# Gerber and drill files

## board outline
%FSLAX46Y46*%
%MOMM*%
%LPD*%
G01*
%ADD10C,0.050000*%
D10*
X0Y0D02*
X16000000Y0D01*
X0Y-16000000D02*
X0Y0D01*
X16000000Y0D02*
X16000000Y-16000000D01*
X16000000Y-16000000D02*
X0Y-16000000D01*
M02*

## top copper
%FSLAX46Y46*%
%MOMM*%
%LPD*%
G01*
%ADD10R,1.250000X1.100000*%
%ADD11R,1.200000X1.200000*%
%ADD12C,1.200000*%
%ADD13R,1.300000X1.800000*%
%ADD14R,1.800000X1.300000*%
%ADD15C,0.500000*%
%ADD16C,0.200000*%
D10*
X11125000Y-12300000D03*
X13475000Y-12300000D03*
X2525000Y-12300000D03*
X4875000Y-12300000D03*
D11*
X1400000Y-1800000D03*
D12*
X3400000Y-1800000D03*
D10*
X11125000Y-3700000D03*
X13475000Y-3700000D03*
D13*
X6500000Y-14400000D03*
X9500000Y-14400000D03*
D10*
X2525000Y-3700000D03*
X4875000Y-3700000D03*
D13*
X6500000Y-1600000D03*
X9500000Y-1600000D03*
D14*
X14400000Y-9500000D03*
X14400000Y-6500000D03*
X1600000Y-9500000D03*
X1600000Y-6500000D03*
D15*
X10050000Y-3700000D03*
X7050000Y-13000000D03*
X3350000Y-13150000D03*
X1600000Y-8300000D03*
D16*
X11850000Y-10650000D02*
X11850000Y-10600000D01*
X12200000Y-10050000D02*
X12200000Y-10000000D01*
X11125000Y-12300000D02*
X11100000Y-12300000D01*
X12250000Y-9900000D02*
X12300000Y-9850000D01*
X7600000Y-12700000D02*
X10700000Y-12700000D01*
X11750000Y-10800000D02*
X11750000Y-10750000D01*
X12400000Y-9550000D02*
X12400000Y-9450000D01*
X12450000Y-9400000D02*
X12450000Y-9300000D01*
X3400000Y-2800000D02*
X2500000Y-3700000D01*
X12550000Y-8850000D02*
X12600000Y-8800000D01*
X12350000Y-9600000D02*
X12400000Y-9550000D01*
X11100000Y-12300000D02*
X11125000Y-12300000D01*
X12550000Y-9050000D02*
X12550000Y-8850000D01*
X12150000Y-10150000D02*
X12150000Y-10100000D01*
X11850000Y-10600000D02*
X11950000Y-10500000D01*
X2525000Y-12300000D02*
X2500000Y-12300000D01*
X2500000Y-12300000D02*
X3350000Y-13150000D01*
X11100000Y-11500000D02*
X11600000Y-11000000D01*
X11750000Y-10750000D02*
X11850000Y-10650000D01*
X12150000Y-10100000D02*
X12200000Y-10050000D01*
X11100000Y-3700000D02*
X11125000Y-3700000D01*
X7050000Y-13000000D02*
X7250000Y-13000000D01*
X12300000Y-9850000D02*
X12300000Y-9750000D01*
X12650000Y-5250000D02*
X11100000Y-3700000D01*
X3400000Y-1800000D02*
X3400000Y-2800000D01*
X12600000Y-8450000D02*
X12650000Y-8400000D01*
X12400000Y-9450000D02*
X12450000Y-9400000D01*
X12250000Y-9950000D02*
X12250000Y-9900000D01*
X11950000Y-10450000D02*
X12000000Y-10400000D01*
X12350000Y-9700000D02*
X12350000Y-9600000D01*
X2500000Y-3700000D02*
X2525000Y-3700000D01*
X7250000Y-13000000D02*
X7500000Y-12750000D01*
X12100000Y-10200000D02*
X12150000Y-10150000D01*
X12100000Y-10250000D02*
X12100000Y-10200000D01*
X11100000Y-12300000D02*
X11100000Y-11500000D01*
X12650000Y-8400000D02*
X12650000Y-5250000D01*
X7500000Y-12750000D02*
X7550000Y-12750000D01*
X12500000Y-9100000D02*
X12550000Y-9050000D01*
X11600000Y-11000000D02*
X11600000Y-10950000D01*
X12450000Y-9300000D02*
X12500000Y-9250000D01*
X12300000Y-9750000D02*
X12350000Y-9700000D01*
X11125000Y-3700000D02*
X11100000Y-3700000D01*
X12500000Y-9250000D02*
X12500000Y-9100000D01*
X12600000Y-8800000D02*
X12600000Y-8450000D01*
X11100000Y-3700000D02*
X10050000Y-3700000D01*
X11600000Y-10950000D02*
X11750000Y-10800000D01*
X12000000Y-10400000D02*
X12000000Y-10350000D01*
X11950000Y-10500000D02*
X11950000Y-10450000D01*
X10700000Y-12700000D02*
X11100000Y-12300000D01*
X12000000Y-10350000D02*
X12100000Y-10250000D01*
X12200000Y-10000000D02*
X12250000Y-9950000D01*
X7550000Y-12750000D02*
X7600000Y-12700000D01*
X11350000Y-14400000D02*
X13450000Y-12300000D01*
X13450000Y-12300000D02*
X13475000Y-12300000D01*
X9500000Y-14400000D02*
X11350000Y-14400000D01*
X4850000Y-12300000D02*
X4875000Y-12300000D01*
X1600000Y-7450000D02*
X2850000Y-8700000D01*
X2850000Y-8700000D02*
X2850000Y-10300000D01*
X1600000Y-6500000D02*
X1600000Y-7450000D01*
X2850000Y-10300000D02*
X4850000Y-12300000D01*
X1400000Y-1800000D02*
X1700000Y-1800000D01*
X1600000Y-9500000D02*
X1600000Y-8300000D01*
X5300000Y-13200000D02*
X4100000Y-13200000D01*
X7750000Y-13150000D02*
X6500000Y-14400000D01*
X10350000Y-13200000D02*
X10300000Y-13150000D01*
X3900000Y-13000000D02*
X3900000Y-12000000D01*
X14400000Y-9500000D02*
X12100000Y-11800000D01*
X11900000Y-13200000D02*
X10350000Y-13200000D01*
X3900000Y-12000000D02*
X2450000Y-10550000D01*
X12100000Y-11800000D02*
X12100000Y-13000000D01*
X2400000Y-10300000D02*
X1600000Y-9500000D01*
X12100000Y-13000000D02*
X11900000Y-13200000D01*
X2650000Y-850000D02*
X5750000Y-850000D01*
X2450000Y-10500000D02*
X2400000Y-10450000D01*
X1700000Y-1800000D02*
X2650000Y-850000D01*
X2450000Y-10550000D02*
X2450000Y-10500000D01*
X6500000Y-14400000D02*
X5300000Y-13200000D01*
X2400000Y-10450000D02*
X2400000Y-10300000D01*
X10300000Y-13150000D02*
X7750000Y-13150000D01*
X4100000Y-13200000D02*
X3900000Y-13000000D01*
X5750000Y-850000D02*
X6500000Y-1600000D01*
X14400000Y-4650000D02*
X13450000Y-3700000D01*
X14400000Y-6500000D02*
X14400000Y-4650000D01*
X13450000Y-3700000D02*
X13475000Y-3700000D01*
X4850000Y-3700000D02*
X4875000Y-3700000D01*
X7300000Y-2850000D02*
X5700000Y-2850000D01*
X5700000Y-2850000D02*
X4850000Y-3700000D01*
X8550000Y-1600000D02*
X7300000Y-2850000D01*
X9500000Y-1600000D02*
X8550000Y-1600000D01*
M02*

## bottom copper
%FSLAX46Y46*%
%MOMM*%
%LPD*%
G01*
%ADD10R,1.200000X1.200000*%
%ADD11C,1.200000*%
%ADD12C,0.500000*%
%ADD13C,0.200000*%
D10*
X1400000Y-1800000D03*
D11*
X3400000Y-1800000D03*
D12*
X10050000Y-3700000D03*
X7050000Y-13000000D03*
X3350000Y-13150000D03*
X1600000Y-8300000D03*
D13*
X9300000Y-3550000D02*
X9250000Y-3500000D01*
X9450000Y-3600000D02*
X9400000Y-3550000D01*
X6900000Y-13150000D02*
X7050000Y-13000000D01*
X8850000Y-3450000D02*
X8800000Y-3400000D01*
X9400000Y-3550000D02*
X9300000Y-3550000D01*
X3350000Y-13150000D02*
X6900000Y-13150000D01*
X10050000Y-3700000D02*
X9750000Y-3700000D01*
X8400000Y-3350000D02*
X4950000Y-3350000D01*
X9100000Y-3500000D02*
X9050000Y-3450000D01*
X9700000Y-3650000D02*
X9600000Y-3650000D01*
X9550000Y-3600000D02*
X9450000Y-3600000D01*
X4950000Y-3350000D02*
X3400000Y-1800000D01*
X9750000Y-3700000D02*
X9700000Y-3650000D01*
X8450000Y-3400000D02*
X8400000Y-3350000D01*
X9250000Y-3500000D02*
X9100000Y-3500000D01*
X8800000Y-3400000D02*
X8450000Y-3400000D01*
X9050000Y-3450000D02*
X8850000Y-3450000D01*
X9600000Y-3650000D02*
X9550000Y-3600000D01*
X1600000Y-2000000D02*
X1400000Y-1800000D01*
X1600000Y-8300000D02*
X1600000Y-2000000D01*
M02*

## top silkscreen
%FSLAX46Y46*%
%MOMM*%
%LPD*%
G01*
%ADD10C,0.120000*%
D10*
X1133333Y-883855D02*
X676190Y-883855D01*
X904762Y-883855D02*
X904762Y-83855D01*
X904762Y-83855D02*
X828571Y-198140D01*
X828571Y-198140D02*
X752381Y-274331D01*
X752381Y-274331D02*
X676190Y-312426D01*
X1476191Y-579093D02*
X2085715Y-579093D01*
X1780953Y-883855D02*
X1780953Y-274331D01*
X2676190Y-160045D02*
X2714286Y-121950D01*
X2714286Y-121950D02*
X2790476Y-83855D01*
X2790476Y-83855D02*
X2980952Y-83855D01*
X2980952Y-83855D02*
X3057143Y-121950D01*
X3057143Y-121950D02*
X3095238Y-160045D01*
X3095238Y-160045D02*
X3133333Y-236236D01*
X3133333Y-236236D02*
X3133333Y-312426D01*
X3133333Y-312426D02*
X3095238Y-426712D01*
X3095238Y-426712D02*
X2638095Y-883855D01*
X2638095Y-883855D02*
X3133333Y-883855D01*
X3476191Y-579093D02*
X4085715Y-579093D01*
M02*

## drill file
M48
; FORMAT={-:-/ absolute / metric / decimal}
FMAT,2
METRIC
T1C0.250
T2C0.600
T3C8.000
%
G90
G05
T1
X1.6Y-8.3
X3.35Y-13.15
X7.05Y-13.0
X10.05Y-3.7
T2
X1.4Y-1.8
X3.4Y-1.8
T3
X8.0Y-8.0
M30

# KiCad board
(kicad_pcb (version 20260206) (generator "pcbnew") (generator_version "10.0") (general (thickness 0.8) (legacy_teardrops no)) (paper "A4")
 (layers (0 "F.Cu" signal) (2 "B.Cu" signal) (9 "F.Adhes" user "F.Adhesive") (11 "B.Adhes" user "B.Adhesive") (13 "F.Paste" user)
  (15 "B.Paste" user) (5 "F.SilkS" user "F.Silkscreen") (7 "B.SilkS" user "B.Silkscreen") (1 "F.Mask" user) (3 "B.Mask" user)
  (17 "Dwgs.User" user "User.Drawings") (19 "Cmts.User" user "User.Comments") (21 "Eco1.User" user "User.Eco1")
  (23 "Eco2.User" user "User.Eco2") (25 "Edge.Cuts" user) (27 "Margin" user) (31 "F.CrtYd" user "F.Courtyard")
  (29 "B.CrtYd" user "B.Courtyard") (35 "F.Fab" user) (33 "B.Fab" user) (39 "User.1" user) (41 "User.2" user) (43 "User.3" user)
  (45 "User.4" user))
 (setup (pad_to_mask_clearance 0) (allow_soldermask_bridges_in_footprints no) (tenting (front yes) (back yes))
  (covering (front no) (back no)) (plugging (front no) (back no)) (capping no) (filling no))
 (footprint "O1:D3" (layer "F.Cu") (at 12.3 12.3)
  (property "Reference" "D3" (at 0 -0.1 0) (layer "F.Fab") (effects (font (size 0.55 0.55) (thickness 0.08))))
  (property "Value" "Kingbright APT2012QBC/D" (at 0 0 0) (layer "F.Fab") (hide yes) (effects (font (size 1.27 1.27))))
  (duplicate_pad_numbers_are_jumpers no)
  (pad "1" smd rect (at -1.175 0) (size 1.25 1.1) (layers "F.Cu" "F.Mask" "F.Paste") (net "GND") (solder_mask_margin 0.025)
   (thermal_bridge_angle 45))
  (pad "2" smd rect (at 1.175 0) (size 1.25 1.1) (layers "F.Cu" "F.Mask" "F.Paste") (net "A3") (solder_mask_margin 0.025)
   (thermal_bridge_angle 45)))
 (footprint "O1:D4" (layer "F.Cu") (at 3.7 12.3)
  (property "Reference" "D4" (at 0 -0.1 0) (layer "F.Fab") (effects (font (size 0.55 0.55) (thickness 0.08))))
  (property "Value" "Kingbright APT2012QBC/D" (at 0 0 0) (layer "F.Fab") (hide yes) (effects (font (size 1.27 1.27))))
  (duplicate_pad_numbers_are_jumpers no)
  (pad "1" smd rect (at -1.175 0) (size 1.25 1.1) (layers "F.Cu" "F.Mask" "F.Paste") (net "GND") (solder_mask_margin 0.025)
   (thermal_bridge_angle 45))
  (pad "2" smd rect (at 1.175 0) (size 1.25 1.1) (layers "F.Cu" "F.Mask" "F.Paste") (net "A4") (solder_mask_margin 0.025)
   (thermal_bridge_angle 45)))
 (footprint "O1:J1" (layer "F.Cu") (at 2.4 1.8)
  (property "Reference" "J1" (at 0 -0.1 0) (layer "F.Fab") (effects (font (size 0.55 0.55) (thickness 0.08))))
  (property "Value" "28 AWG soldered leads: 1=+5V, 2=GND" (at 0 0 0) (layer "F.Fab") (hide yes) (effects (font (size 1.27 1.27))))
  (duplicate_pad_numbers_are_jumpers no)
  (pad "1" thru_hole rect (at -1 0) (size 1.2 1.2) (drill 0.6) (layers "*.Cu" "*.Mask") (remove_unused_layers no) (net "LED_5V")
   (solder_mask_margin 0.025) (thermal_bridge_angle 45))
  (pad "2" thru_hole circle (at 1 0) (size 1.2 1.2) (drill 0.6) (layers "*.Cu" "*.Mask") (remove_unused_layers no) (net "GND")
   (solder_mask_margin 0.025)))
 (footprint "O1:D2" (layer "F.Cu") (at 12.3 3.7)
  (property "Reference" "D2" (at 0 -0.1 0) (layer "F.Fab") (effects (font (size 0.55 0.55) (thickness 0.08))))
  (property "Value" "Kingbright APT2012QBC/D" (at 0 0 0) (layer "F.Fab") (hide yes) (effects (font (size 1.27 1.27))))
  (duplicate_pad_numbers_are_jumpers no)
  (pad "1" smd rect (at -1.175 0) (size 1.25 1.1) (layers "F.Cu" "F.Mask" "F.Paste") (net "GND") (solder_mask_margin 0.025)
   (thermal_bridge_angle 45))
  (pad "2" smd rect (at 1.175 0) (size 1.25 1.1) (layers "F.Cu" "F.Mask" "F.Paste") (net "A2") (solder_mask_margin 0.025)
   (thermal_bridge_angle 45)))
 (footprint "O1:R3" (layer "F.Cu") (at 8 14.4)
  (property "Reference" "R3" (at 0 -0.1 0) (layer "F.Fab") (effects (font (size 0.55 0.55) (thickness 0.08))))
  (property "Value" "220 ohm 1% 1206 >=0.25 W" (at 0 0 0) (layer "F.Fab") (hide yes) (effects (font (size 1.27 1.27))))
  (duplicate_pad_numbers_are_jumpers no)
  (pad "1" smd rect (at -1.5 0) (size 1.3 1.8) (layers "F.Cu" "F.Mask" "F.Paste") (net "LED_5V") (solder_mask_margin 0.025)
   (thermal_bridge_angle 45))
  (pad "2" smd rect (at 1.5 0) (size 1.3 1.8) (layers "F.Cu" "F.Mask" "F.Paste") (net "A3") (solder_mask_margin 0.025)
   (thermal_bridge_angle 45)))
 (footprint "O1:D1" (layer "F.Cu") (at 3.7 3.7)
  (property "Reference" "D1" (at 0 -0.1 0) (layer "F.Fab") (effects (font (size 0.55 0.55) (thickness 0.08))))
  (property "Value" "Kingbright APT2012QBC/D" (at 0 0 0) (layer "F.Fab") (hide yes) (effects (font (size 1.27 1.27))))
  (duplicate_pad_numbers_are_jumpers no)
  (pad "1" smd rect (at -1.175 0) (size 1.25 1.1) (layers "F.Cu" "F.Mask" "F.Paste") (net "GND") (solder_mask_margin 0.025)
   (thermal_bridge_angle 45))
  (pad "2" smd rect (at 1.175 0) (size 1.25 1.1) (layers "F.Cu" "F.Mask" "F.Paste") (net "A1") (solder_mask_margin 0.025)
   (thermal_bridge_angle 45)))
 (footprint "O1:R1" (layer "F.Cu") (at 8 1.6)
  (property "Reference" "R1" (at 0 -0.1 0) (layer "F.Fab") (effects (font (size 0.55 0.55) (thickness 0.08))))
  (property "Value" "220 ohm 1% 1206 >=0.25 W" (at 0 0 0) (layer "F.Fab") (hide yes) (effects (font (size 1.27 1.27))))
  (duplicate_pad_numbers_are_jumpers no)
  (pad "1" smd rect (at -1.5 0) (size 1.3 1.8) (layers "F.Cu" "F.Mask" "F.Paste") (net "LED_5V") (solder_mask_margin 0.025)
   (thermal_bridge_angle 45))
  (pad "2" smd rect (at 1.5 0) (size 1.3 1.8) (layers "F.Cu" "F.Mask" "F.Paste") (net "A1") (solder_mask_margin 0.025)
   (thermal_bridge_angle 45)))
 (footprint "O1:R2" (layer "F.Cu") (at 14.4 8 90)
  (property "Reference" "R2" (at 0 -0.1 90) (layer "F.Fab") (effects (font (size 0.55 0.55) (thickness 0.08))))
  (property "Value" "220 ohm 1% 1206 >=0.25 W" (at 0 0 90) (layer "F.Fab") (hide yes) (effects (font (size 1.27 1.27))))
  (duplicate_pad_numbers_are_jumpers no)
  (pad "1" smd rect (at -1.5 0 90) (size 1.3 1.8) (layers "F.Cu" "F.Mask" "F.Paste") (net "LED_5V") (solder_mask_margin 0.025)
   (thermal_bridge_angle 45))
  (pad "2" smd rect (at 1.5 0 90) (size 1.3 1.8) (layers "F.Cu" "F.Mask" "F.Paste") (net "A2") (solder_mask_margin 0.025)
   (thermal_bridge_angle 45)))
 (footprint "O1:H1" (layer "F.Cu") (at 8 8)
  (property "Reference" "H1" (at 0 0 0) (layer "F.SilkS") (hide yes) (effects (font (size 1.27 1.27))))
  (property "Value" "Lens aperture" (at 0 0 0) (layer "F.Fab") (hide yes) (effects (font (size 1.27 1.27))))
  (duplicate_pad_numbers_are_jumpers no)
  (pad "" np_thru_hole circle (at 0 0) (size 8 8) (drill 8) (layers "*.Cu" "*.Mask")))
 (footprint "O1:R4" (layer "F.Cu") (at 1.6 8 90)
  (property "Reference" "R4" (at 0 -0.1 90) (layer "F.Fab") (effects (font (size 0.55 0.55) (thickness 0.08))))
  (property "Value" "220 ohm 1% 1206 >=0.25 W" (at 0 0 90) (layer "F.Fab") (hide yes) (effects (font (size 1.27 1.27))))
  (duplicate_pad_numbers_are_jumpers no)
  (pad "1" smd rect (at -1.5 0 90) (size 1.3 1.8) (layers "F.Cu" "F.Mask" "F.Paste") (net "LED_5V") (solder_mask_margin 0.025)
   (thermal_bridge_angle 45))
  (pad "2" smd rect (at 1.5 0 90) (size 1.3 1.8) (layers "F.Cu" "F.Mask" "F.Paste") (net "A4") (solder_mask_margin 0.025)
   (thermal_bridge_angle 45)))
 (gr_line (start 0 0) (end 16 0) (stroke (width 0.05) (type default)) (layer "Edge.Cuts"))
 (gr_line (start 0 16) (end 0 0) (stroke (width 0.05) (type default)) (layer "Edge.Cuts"))
 (gr_line (start 16 0) (end 16 16) (stroke (width 0.05) (type default)) (layer "Edge.Cuts"))
 (gr_line (start 16 16) (end 0 16) (stroke (width 0.05) (type default)) (layer "Edge.Cuts"))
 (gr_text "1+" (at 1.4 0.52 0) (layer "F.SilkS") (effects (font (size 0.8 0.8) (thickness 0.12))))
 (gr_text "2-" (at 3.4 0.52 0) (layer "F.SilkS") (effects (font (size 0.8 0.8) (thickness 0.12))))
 (segment (start 11.85 10.65) (end 11.85 10.6) (width 0.2) (layer "F.Cu") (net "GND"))
 (segment (start 12.2 10.05) (end 12.2 10) (width 0.2) (layer "F.Cu") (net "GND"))
 (segment (start 11.125 12.3) (end 11.1 12.3) (width 0.2) (layer "F.Cu") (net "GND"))
 (segment (start 12.25 9.9) (end 12.3 9.85) (width 0.2) (layer "F.Cu") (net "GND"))
 (segment (start 7.6 12.7) (end 10.7 12.7) (width 0.2) (layer "F.Cu") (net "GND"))
 (segment (start 11.75 10.8) (end 11.75 10.75) (width 0.2) (layer "F.Cu") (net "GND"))
 (segment (start 12.4 9.55) (end 12.4 9.45) (width 0.2) (layer "F.Cu") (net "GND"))
 (segment (start 12.45 9.4) (end 12.45 9.3) (width 0.2) (layer "F.Cu") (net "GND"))
 (segment (start 3.4 2.8) (end 2.5 3.7) (width 0.2) (layer "F.Cu") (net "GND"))
 (segment (start 12.55 8.85) (end 12.6 8.8) (width 0.2) (layer "F.Cu") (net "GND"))
 (segment (start 12.35 9.6) (end 12.4 9.55) (width 0.2) (layer "F.Cu") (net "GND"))
 (segment (start 11.1 12.3) (end 11.125 12.3) (width 0.2) (layer "F.Cu") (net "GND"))
 (segment (start 12.55 9.05) (end 12.55 8.85) (width 0.2) (layer "F.Cu") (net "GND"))
 (segment (start 12.15 10.15) (end 12.15 10.1) (width 0.2) (layer "F.Cu") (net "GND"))
 (segment (start 11.85 10.6) (end 11.95 10.5) (width 0.2) (layer "F.Cu") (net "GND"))
 (segment (start 2.525 12.3) (end 2.5 12.3) (width 0.2) (layer "F.Cu") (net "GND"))
 (segment (start 2.5 12.3) (end 3.35 13.15) (width 0.2) (layer "F.Cu") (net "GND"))
 (segment (start 11.1 11.5) (end 11.6 11) (width 0.2) (layer "F.Cu") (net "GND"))
 (segment (start 11.75 10.75) (end 11.85 10.65) (width 0.2) (layer "F.Cu") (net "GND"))
 (segment (start 12.15 10.1) (end 12.2 10.05) (width 0.2) (layer "F.Cu") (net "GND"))
 (segment (start 11.1 3.7) (end 11.125 3.7) (width 0.2) (layer "F.Cu") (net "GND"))
 (segment (start 7.05 13) (end 7.25 13) (width 0.2) (layer "F.Cu") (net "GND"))
 (segment (start 12.3 9.85) (end 12.3 9.75) (width 0.2) (layer "F.Cu") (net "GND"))
 (segment (start 12.65 5.25) (end 11.1 3.7) (width 0.2) (layer "F.Cu") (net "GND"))
 (segment (start 3.4 1.8) (end 3.4 2.8) (width 0.2) (layer "F.Cu") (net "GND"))
 (segment (start 12.6 8.45) (end 12.65 8.4) (width 0.2) (layer "F.Cu") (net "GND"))
 (segment (start 12.4 9.45) (end 12.45 9.4) (width 0.2) (layer "F.Cu") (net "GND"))
 (segment (start 12.25 9.95) (end 12.25 9.9) (width 0.2) (layer "F.Cu") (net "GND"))
 (segment (start 11.95 10.45) (end 12 10.4) (width 0.2) (layer "F.Cu") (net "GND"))
 (segment (start 12.35 9.7) (end 12.35 9.6) (width 0.2) (layer "F.Cu") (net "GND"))
 (segment (start 2.5 3.7) (end 2.525 3.7) (width 0.2) (layer "F.Cu") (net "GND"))
 (segment (start 7.25 13) (end 7.5 12.75) (width 0.2) (layer "F.Cu") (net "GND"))
 (segment (start 12.1 10.2) (end 12.15 10.15) (width 0.2) (layer "F.Cu") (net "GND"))
 (segment (start 12.1 10.25) (end 12.1 10.2) (width 0.2) (layer "F.Cu") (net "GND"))
 (segment (start 11.1 12.3) (end 11.1 11.5) (width 0.2) (layer "F.Cu") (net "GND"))
 (segment (start 12.65 8.4) (end 12.65 5.25) (width 0.2) (layer "F.Cu") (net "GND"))
 (segment (start 7.5 12.75) (end 7.55 12.75) (width 0.2) (layer "F.Cu") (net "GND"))
 (segment (start 12.5 9.1) (end 12.55 9.05) (width 0.2) (layer "F.Cu") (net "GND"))
 (segment (start 11.6 11) (end 11.6 10.95) (width 0.2) (layer "F.Cu") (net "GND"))
 (segment (start 12.45 9.3) (end 12.5 9.25) (width 0.2) (layer "F.Cu") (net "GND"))
 (segment (start 12.3 9.75) (end 12.35 9.7) (width 0.2) (layer "F.Cu") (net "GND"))
 (segment (start 11.125 3.7) (end 11.1 3.7) (width 0.2) (layer "F.Cu") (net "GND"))
 (segment (start 12.5 9.25) (end 12.5 9.1) (width 0.2) (layer "F.Cu") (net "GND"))
 (segment (start 12.6 8.8) (end 12.6 8.45) (width 0.2) (layer "F.Cu") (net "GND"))
 (segment (start 11.1 3.7) (end 10.05 3.7) (width 0.2) (layer "F.Cu") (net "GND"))
 (segment (start 11.6 10.95) (end 11.75 10.8) (width 0.2) (layer "F.Cu") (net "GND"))
 (segment (start 12 10.4) (end 12 10.35) (width 0.2) (layer "F.Cu") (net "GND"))
 (segment (start 11.95 10.5) (end 11.95 10.45) (width 0.2) (layer "F.Cu") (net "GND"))
 (segment (start 10.7 12.7) (end 11.1 12.3) (width 0.2) (layer "F.Cu") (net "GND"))
 (segment (start 12 10.35) (end 12.1 10.25) (width 0.2) (layer "F.Cu") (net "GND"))
 (segment (start 12.2 10) (end 12.25 9.95) (width 0.2) (layer "F.Cu") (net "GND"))
 (segment (start 7.55 12.75) (end 7.6 12.7) (width 0.2) (layer "F.Cu") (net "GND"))
 (via (at 10.05 3.7) (size 0.5) (drill 0.25) (layers "F.Cu" "B.Cu") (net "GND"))
 (via (at 7.05 13) (size 0.5) (drill 0.25) (layers "F.Cu" "B.Cu") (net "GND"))
 (via (at 3.35 13.15) (size 0.5) (drill 0.25) (layers "F.Cu" "B.Cu") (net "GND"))
 (segment (start 9.3 3.55) (end 9.25 3.5) (width 0.2) (layer "B.Cu") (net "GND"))
 (segment (start 9.45 3.6) (end 9.4 3.55) (width 0.2) (layer "B.Cu") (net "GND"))
 (segment (start 6.9 13.15) (end 7.05 13) (width 0.2) (layer "B.Cu") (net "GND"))
 (segment (start 8.85 3.45) (end 8.8 3.4) (width 0.2) (layer "B.Cu") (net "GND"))
 (segment (start 9.4 3.55) (end 9.3 3.55) (width 0.2) (layer "B.Cu") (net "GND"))
 (segment (start 3.35 13.15) (end 6.9 13.15) (width 0.2) (layer "B.Cu") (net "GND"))
 (segment (start 10.05 3.7) (end 9.75 3.7) (width 0.2) (layer "B.Cu") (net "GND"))
 (segment (start 8.4 3.35) (end 4.95 3.35) (width 0.2) (layer "B.Cu") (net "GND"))
 (segment (start 9.1 3.5) (end 9.05 3.45) (width 0.2) (layer "B.Cu") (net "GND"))
 (segment (start 9.7 3.65) (end 9.6 3.65) (width 0.2) (layer "B.Cu") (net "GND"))
 (segment (start 9.55 3.6) (end 9.45 3.6) (width 0.2) (layer "B.Cu") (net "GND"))
 (segment (start 4.95 3.35) (end 3.4 1.8) (width 0.2) (layer "B.Cu") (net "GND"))
 (segment (start 9.75 3.7) (end 9.7 3.65) (width 0.2) (layer "B.Cu") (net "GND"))
 (segment (start 8.45 3.4) (end 8.4 3.35) (width 0.2) (layer "B.Cu") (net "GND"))
 (segment (start 9.25 3.5) (end 9.1 3.5) (width 0.2) (layer "B.Cu") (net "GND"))
 (segment (start 8.8 3.4) (end 8.45 3.4) (width 0.2) (layer "B.Cu") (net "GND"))
 (segment (start 9.05 3.45) (end 8.85 3.45) (width 0.2) (layer "B.Cu") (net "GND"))
 (segment (start 9.6 3.65) (end 9.55 3.6) (width 0.2) (layer "B.Cu") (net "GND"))
 (segment (start 11.35 14.4) (end 13.45 12.3) (width 0.2) (layer "F.Cu") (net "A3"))
 (segment (start 13.45 12.3) (end 13.475 12.3) (width 0.2) (layer "F.Cu") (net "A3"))
 (segment (start 9.5 14.4) (end 11.35 14.4) (width 0.2) (layer "F.Cu") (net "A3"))
 (segment (start 4.85 12.3) (end 4.875 12.3) (width 0.2) (layer "F.Cu") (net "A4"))
 (segment (start 1.6 7.45) (end 2.85 8.7) (width 0.2) (layer "F.Cu") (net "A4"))
 (segment (start 2.85 8.7) (end 2.85 10.3) (width 0.2) (layer "F.Cu") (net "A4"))
 (segment (start 1.6 6.5) (end 1.6 7.45) (width 0.2) (layer "F.Cu") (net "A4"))
 (segment (start 2.85 10.3) (end 4.85 12.3) (width 0.2) (layer "F.Cu") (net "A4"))
 (segment (start 1.4 1.8) (end 1.7 1.8) (width 0.2) (layer "F.Cu") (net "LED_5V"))
 (segment (start 1.6 9.5) (end 1.6 8.3) (width 0.2) (layer "F.Cu") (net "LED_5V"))
 (segment (start 5.3 13.2) (end 4.1 13.2) (width 0.2) (layer "F.Cu") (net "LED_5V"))
 (segment (start 7.75 13.15) (end 6.5 14.4) (width 0.2) (layer "F.Cu") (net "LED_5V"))
 (segment (start 10.35 13.2) (end 10.3 13.15) (width 0.2) (layer "F.Cu") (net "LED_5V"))
 (segment (start 3.9 13) (end 3.9 12) (width 0.2) (layer "F.Cu") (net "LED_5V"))
 (segment (start 14.4 9.5) (end 12.1 11.8) (width 0.2) (layer "F.Cu") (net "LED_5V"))
 (segment (start 11.9 13.2) (end 10.35 13.2) (width 0.2) (layer "F.Cu") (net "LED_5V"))
 (segment (start 3.9 12) (end 2.45 10.55) (width 0.2) (layer "F.Cu") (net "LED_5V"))
 (segment (start 12.1 11.8) (end 12.1 13) (width 0.2) (layer "F.Cu") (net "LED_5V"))
 (segment (start 2.4 10.3) (end 1.6 9.5) (width 0.2) (layer "F.Cu") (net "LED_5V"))
 (segment (start 12.1 13) (end 11.9 13.2) (width 0.2) (layer "F.Cu") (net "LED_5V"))
 (segment (start 2.65 0.85) (end 5.75 0.85) (width 0.2) (layer "F.Cu") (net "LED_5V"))
 (segment (start 2.45 10.5) (end 2.4 10.45) (width 0.2) (layer "F.Cu") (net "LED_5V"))
 (segment (start 1.7 1.8) (end 2.65 0.85) (width 0.2) (layer "F.Cu") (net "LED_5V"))
 (segment (start 2.45 10.55) (end 2.45 10.5) (width 0.2) (layer "F.Cu") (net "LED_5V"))
 (segment (start 6.5 14.4) (end 5.3 13.2) (width 0.2) (layer "F.Cu") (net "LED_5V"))
 (segment (start 2.4 10.45) (end 2.4 10.3) (width 0.2) (layer "F.Cu") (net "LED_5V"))
 (segment (start 10.3 13.15) (end 7.75 13.15) (width 0.2) (layer "F.Cu") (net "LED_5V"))
 (segment (start 4.1 13.2) (end 3.9 13) (width 0.2) (layer "F.Cu") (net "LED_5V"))
 (segment (start 5.75 0.85) (end 6.5 1.6) (width 0.2) (layer "F.Cu") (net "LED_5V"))
 (via (at 1.6 8.3) (size 0.5) (drill 0.25) (layers "F.Cu" "B.Cu") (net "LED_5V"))
 (segment (start 1.6 2) (end 1.4 1.8) (width 0.2) (layer "B.Cu") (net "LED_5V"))
 (segment (start 1.6 8.3) (end 1.6 2) (width 0.2) (layer "B.Cu") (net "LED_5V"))
 (segment (start 14.4 4.65) (end 13.45 3.7) (width 0.2) (layer "F.Cu") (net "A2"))
 (segment (start 14.4 6.5) (end 14.4 4.65) (width 0.2) (layer "F.Cu") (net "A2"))
 (segment (start 13.45 3.7) (end 13.475 3.7) (width 0.2) (layer "F.Cu") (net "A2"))
 (segment (start 4.85 3.7) (end 4.875 3.7) (width 0.2) (layer "F.Cu") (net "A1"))
 (segment (start 7.3 2.85) (end 5.7 2.85) (width 0.2) (layer "F.Cu") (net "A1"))
 (segment (start 5.7 2.85) (end 4.85 3.7) (width 0.2) (layer "F.Cu") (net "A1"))
 (segment (start 8.55 1.6) (end 7.3 2.85) (width 0.2) (layer "F.Cu") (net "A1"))
 (segment (start 9.5 1.6) (end 8.55 1.6) (width 0.2) (layer "F.Cu") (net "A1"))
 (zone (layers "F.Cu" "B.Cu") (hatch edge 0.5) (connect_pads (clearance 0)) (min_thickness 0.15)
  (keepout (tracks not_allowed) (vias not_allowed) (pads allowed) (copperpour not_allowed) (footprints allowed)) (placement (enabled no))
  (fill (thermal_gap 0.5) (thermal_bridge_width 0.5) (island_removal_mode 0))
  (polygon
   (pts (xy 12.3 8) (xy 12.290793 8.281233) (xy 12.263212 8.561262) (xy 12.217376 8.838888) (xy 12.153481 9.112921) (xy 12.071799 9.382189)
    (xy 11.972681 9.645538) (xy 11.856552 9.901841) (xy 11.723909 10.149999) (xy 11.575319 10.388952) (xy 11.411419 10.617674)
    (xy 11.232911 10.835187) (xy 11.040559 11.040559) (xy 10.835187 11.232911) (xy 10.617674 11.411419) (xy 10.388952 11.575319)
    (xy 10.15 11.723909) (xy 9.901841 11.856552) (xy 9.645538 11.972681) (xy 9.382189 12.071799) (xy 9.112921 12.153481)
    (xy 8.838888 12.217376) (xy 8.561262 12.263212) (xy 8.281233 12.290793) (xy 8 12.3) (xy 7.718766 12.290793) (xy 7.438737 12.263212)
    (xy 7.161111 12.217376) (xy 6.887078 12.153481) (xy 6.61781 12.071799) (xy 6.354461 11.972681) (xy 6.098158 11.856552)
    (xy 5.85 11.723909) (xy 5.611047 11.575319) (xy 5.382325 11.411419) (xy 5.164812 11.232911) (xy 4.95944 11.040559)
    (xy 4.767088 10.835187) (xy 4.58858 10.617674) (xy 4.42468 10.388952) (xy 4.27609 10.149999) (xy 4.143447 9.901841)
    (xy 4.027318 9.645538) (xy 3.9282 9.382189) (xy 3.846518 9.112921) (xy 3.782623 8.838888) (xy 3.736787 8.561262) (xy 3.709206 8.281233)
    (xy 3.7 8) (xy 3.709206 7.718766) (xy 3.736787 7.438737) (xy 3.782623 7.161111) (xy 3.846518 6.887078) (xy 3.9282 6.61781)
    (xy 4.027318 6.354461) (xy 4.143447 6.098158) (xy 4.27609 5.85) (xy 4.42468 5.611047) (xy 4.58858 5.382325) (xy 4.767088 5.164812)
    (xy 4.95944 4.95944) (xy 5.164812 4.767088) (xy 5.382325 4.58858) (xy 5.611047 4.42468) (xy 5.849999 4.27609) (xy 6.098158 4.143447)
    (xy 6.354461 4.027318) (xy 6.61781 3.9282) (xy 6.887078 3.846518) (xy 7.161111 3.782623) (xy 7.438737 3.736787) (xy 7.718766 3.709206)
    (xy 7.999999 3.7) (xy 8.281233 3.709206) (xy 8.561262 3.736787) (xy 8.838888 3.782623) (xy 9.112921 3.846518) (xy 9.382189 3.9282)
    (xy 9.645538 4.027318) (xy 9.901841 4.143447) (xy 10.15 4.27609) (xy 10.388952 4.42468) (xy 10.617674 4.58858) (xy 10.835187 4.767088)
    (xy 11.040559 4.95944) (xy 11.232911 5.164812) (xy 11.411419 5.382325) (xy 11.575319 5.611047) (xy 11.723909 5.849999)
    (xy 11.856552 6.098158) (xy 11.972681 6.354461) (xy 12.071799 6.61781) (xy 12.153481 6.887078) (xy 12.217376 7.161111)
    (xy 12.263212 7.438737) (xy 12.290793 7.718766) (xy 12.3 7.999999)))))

